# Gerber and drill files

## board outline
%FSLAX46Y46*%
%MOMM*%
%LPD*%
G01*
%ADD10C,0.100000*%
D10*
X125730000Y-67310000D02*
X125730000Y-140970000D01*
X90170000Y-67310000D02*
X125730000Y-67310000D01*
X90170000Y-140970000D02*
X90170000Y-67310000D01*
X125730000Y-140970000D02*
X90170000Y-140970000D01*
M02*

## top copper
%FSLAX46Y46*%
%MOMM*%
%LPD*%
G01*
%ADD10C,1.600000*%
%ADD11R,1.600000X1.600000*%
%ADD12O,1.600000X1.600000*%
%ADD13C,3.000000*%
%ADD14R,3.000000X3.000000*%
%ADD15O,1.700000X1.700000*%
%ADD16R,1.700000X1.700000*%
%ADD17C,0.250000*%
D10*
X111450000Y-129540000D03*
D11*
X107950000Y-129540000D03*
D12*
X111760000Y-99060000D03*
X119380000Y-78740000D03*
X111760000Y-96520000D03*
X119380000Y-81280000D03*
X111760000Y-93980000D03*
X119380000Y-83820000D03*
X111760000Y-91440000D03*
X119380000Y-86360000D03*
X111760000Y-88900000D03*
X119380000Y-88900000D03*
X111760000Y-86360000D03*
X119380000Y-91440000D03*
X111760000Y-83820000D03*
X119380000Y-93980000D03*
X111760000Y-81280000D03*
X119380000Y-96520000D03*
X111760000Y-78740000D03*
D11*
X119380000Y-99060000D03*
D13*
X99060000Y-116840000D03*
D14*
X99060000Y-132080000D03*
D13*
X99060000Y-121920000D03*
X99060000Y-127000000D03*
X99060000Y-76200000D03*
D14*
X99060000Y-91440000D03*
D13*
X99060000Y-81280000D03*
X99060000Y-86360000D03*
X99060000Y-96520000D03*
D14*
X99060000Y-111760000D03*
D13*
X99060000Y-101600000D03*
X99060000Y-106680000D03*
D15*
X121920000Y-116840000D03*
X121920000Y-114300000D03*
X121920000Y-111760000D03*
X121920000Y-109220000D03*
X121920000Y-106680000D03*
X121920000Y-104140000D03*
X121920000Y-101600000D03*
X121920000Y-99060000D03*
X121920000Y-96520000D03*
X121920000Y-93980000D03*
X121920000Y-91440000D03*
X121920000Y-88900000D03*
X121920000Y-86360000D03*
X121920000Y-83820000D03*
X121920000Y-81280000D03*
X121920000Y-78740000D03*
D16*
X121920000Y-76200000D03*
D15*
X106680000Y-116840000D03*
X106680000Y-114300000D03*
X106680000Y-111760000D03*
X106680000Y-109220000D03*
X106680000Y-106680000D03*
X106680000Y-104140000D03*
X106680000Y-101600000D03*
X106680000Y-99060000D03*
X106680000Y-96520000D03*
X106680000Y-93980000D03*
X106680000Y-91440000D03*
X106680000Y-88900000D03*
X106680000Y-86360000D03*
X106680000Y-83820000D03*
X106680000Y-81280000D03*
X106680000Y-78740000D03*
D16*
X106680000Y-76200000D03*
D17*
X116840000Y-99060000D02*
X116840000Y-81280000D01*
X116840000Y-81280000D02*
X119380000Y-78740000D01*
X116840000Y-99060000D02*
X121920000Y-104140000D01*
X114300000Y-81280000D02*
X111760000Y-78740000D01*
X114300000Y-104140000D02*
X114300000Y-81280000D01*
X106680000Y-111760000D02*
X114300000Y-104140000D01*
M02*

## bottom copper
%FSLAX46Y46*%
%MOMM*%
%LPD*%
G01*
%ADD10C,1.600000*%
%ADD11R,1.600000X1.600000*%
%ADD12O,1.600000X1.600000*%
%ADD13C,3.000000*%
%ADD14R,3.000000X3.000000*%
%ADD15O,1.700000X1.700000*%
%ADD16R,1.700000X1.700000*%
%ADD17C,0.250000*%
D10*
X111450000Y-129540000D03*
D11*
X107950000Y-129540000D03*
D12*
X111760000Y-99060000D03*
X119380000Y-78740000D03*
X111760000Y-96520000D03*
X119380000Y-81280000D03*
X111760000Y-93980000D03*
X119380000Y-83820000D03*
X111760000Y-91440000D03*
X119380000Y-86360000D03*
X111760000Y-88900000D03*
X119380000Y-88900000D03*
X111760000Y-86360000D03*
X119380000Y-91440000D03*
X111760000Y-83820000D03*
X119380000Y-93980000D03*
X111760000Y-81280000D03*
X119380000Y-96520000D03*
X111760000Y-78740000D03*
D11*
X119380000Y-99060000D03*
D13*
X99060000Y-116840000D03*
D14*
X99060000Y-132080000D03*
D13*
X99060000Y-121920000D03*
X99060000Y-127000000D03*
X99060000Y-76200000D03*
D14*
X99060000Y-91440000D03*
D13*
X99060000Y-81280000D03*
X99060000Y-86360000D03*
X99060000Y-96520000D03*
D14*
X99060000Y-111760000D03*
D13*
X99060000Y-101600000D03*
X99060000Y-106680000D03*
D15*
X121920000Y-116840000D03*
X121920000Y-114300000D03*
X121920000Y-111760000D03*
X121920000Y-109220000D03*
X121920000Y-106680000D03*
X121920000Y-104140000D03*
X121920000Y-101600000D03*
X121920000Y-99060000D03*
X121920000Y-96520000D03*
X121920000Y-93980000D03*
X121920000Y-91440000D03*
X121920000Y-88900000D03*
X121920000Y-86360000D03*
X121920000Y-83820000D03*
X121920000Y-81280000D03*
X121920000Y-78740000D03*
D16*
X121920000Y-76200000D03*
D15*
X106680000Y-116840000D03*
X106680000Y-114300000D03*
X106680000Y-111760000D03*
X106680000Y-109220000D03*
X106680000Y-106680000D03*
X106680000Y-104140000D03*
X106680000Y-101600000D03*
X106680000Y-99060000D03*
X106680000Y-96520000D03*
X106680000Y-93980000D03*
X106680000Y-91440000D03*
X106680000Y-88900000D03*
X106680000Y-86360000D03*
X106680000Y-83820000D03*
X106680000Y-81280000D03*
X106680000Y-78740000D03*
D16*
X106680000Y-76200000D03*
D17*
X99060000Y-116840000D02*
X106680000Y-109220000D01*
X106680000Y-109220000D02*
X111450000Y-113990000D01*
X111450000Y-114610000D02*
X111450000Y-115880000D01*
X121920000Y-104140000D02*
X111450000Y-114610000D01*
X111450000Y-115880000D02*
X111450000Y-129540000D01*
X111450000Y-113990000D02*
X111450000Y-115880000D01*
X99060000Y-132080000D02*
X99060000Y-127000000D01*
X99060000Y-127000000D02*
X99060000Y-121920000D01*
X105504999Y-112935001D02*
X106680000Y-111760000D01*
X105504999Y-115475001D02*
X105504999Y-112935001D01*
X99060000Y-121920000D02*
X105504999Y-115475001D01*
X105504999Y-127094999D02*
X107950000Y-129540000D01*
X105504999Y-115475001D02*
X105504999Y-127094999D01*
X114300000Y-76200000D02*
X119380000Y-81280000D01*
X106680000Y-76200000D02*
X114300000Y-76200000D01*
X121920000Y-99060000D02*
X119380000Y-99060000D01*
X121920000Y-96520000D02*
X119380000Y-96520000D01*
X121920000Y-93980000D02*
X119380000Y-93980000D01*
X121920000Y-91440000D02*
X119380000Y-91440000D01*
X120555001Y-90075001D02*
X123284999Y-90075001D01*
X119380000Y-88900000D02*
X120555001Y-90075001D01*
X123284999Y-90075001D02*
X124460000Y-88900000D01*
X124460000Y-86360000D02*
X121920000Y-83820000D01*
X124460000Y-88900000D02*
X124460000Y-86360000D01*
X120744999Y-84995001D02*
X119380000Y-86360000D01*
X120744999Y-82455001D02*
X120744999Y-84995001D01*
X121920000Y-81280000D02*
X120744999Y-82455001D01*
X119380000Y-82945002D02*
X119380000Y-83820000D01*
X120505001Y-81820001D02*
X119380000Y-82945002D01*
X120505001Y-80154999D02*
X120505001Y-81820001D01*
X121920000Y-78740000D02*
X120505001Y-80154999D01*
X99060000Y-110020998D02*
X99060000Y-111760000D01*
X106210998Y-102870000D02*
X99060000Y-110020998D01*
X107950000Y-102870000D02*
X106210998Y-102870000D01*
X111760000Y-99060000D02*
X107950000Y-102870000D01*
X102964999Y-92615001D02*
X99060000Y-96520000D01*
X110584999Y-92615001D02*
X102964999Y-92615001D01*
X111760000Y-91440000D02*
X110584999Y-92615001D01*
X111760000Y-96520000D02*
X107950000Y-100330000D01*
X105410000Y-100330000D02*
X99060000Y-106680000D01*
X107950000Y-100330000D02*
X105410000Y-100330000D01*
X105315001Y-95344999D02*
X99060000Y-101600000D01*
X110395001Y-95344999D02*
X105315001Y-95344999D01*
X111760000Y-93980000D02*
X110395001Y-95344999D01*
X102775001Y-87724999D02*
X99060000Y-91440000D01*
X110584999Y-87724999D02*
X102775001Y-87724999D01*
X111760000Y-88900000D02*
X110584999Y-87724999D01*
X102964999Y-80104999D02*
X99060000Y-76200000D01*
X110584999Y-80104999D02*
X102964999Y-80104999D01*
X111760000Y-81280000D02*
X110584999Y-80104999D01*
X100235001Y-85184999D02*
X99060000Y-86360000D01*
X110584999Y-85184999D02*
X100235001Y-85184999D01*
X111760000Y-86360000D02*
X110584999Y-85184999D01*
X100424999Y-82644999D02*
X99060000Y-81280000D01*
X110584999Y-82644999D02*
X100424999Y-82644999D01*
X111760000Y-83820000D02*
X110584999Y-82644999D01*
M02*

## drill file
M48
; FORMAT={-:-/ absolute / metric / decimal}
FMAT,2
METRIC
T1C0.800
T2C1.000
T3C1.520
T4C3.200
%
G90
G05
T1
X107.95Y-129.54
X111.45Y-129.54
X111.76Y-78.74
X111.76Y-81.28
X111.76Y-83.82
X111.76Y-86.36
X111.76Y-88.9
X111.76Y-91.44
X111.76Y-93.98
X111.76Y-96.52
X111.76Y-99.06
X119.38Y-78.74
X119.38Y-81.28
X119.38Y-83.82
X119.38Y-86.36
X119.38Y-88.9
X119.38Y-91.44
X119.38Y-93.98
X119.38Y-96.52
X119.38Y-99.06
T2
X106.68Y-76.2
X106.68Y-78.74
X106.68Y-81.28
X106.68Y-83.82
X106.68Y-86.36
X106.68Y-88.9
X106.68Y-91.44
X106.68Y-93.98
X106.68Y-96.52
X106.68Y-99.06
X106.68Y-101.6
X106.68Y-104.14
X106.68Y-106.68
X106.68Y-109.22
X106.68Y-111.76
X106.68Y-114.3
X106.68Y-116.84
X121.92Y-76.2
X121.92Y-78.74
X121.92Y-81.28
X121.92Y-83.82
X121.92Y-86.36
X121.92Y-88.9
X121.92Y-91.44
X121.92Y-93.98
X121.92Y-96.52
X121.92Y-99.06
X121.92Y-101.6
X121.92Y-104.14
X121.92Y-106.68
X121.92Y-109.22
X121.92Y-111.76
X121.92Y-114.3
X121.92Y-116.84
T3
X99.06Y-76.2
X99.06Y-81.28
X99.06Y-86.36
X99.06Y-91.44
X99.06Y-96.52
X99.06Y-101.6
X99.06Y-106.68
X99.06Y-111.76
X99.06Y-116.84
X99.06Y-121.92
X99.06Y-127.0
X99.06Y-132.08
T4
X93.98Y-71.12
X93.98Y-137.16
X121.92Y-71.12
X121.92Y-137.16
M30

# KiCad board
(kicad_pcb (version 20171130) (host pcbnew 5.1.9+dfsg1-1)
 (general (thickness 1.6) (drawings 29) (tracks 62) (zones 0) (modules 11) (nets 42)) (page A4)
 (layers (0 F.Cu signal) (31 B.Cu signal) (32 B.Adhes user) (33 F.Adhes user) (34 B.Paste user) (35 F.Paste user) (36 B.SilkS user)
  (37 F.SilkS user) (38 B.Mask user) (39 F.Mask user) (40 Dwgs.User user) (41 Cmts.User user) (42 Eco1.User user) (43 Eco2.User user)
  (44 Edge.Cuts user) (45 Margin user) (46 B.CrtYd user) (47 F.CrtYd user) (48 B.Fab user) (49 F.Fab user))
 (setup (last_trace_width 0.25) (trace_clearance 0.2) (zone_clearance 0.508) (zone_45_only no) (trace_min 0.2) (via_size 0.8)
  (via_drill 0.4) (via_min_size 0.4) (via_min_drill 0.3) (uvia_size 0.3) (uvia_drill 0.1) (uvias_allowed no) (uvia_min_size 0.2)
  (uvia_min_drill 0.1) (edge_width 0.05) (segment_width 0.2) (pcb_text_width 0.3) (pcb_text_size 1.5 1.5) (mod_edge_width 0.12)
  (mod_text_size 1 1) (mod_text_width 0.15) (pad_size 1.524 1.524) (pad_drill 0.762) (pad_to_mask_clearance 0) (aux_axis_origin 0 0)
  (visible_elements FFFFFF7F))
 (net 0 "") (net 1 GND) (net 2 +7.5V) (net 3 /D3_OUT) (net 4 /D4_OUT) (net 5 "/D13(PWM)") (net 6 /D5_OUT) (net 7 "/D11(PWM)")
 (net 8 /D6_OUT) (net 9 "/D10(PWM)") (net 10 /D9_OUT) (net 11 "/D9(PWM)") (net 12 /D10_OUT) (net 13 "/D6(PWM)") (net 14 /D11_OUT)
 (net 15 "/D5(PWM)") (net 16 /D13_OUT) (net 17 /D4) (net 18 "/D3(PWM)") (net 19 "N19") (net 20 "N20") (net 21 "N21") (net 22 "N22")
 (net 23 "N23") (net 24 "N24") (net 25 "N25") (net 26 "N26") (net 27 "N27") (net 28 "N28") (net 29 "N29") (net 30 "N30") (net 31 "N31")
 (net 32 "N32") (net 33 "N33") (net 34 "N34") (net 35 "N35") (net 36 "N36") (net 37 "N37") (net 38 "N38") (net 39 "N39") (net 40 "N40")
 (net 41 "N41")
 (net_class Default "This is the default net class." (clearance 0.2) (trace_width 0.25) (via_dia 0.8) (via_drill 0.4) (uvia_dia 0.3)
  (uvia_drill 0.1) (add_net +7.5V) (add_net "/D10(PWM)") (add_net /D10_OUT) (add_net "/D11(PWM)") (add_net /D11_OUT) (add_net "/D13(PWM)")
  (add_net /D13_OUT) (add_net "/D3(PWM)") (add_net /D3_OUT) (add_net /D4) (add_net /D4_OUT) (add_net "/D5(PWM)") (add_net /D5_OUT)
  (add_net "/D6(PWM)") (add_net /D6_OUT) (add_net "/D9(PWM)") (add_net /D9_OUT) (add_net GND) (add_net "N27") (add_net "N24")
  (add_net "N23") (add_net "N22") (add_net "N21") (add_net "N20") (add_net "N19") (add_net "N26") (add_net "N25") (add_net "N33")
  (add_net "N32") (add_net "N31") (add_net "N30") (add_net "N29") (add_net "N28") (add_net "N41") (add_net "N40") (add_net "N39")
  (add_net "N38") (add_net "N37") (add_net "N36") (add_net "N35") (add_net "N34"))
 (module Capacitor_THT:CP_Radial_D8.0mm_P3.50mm (layer F.Cu) (at 107.95 129.54)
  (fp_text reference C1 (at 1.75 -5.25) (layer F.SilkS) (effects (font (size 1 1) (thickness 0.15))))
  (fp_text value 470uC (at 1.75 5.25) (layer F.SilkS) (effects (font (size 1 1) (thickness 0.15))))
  (pad 2 thru_hole circle (at 3.5 0) (size 1.6 1.6) (drill 0.8) (layers *.Cu *.Mask) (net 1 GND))
  (pad 1 thru_hole rect (at 0 0) (size 1.6 1.6) (drill 0.8) (layers *.Cu *.Mask) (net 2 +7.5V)))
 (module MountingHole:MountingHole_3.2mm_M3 (layer F.Cu) (at 121.92 137.16)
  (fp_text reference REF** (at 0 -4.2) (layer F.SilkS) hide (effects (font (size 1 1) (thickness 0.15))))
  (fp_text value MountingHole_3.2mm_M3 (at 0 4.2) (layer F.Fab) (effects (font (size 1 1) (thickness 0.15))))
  (pad 1 np_thru_hole circle (at 0 0) (size 3.2 3.2) (drill 3.2) (layers *.Cu *.Mask)))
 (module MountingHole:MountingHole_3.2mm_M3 (layer F.Cu) (at 93.98 137.16)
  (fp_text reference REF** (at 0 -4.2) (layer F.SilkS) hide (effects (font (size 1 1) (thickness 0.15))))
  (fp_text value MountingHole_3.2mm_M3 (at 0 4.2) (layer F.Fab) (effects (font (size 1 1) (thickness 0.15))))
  (pad 1 np_thru_hole circle (at 0 0) (size 3.2 3.2) (drill 3.2) (layers *.Cu *.Mask)))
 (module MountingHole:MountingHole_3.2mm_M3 (layer F.Cu) (at 121.92 71.12)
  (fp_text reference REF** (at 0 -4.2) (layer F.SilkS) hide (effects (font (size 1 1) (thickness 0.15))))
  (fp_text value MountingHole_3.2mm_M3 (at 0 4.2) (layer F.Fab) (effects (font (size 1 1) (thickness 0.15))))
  (pad 1 np_thru_hole circle (at 0 0) (size 3.2 3.2) (drill 3.2) (layers *.Cu *.Mask)))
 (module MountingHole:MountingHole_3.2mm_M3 (layer F.Cu) (at 93.98 71.12)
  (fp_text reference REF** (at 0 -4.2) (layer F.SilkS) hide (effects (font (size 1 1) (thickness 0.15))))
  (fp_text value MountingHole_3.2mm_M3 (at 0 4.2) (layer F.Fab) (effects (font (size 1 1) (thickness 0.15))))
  (pad 1 np_thru_hole circle (at 0 0) (size 3.2 3.2) (drill 3.2) (layers *.Cu *.Mask)))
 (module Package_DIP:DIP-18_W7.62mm (layer F.Cu) (at 119.38 99.06 180)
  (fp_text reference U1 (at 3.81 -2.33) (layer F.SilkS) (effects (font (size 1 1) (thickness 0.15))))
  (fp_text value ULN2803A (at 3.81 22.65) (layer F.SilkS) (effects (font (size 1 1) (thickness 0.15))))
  (pad 18 thru_hole oval (at 7.62 0 180) (size 1.6 1.6) (drill 0.8) (layers *.Cu *.Mask) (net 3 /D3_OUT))
  (pad 9 thru_hole oval (at 0 20.32 180) (size 1.6 1.6) (drill 0.8) (layers *.Cu *.Mask) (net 1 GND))
  (pad 17 thru_hole oval (at 7.62 2.54 180) (size 1.6 1.6) (drill 0.8) (layers *.Cu *.Mask) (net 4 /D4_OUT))
  (pad 8 thru_hole oval (at 0 17.78 180) (size 1.6 1.6) (drill 0.8) (layers *.Cu *.Mask) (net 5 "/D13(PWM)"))
  (pad 16 thru_hole oval (at 7.62 5.08 180) (size 1.6 1.6) (drill 0.8) (layers *.Cu *.Mask) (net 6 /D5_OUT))
  (pad 7 thru_hole oval (at 0 15.24 180) (size 1.6 1.6) (drill 0.8) (layers *.Cu *.Mask) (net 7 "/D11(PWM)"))
  (pad 15 thru_hole oval (at 7.62 7.62 180) (size 1.6 1.6) (drill 0.8) (layers *.Cu *.Mask) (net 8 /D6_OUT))
  (pad 6 thru_hole oval (at 0 12.7 180) (size 1.6 1.6) (drill 0.8) (layers *.Cu *.Mask) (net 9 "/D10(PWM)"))
  (pad 14 thru_hole oval (at 7.62 10.16 180) (size 1.6 1.6) (drill 0.8) (layers *.Cu *.Mask) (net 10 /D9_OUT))
  (pad 5 thru_hole oval (at 0 10.16 180) (size 1.6 1.6) (drill 0.8) (layers *.Cu *.Mask) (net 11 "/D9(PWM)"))
  (pad 13 thru_hole oval (at 7.62 12.7 180) (size 1.6 1.6) (drill 0.8) (layers *.Cu *.Mask) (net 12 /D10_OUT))
  (pad 4 thru_hole oval (at 0 7.62 180) (size 1.6 1.6) (drill 0.8) (layers *.Cu *.Mask) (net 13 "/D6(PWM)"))
  (pad 12 thru_hole oval (at 7.62 15.24 180) (size 1.6 1.6) (drill 0.8) (layers *.Cu *.Mask) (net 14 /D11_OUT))
  (pad 3 thru_hole oval (at 0 5.08 180) (size 1.6 1.6) (drill 0.8) (layers *.Cu *.Mask) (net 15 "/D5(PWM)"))
  (pad 11 thru_hole oval (at 7.62 17.78 180) (size 1.6 1.6) (drill 0.8) (layers *.Cu *.Mask) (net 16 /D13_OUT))
  (pad 2 thru_hole oval (at 0 2.54 180) (size 1.6 1.6) (drill 0.8) (layers *.Cu *.Mask) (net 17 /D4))
  (pad 10 thru_hole oval (at 7.62 20.32 180) (size 1.6 1.6) (drill 0.8) (layers *.Cu *.Mask) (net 2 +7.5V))
  (pad 1 thru_hole rect (at 0 0 180) (size 1.6 1.6) (drill 0.8) (layers *.Cu *.Mask) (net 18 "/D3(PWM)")))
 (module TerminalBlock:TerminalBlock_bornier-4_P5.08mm (layer F.Cu) (at 99.06 132.08 90)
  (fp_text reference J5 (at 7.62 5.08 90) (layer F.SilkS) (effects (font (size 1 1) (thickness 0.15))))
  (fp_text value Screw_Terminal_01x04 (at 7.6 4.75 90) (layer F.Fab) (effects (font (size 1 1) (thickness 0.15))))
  (pad 4 thru_hole circle (at 15.24 0 90) (size 3 3) (drill 1.52) (layers *.Cu *.Mask) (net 1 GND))
  (pad 1 thru_hole rect (at 0 0 90) (size 3 3) (drill 1.52) (layers *.Cu *.Mask) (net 2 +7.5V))
  (pad 3 thru_hole circle (at 10.16 0 90) (size 3 3) (drill 1.52) (layers *.Cu *.Mask) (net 2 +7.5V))
  (pad 2 thru_hole circle (at 5.08 0 90) (size 3 3) (drill 1.52) (layers *.Cu *.Mask) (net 2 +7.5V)))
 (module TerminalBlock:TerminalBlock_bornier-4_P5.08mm (layer F.Cu) (at 99.06 91.44 90)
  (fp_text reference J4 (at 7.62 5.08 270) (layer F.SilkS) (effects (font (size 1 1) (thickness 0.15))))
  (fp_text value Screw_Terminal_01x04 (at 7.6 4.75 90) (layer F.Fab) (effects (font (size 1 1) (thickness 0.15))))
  (pad 4 thru_hole circle (at 15.24 0 90) (size 3 3) (drill 1.52) (layers *.Cu *.Mask) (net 16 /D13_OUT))
  (pad 1 thru_hole rect (at 0 0 90) (size 3 3) (drill 1.52) (layers *.Cu *.Mask) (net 10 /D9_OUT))
  (pad 3 thru_hole circle (at 10.16 0 90) (size 3 3) (drill 1.52) (layers *.Cu *.Mask) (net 14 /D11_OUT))
  (pad 2 thru_hole circle (at 5.08 0 90) (size 3 3) (drill 1.52) (layers *.Cu *.Mask) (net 12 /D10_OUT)))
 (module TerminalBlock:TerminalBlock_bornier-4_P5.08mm (layer F.Cu) (at 99.06 111.76 90)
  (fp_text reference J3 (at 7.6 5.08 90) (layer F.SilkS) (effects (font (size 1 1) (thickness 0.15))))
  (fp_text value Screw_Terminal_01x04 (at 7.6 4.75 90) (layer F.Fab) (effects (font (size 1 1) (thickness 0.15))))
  (pad 4 thru_hole circle (at 15.24 0 90) (size 3 3) (drill 1.52) (layers *.Cu *.Mask) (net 8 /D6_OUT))
  (pad 1 thru_hole rect (at 0 0 90) (size 3 3) (drill 1.52) (layers *.Cu *.Mask) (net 3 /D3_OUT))
  (pad 3 thru_hole circle (at 10.16 0 90) (size 3 3) (drill 1.52) (layers *.Cu *.Mask) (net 6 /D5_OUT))
  (pad 2 thru_hole circle (at 5.08 0 90) (size 3 3) (drill 1.52) (layers *.Cu *.Mask) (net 4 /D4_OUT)))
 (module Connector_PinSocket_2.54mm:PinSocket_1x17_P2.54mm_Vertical (layer F.Cu) (at 121.92 76.2)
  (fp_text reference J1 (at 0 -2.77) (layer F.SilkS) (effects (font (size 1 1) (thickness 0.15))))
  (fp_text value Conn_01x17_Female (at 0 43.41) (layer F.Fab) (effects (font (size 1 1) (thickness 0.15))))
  (pad 17 thru_hole oval (at 0 40.64) (size 1.7 1.7) (drill 1) (layers *.Cu *.Mask) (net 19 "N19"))
  (pad 16 thru_hole oval (at 0 38.1) (size 1.7 1.7) (drill 1) (layers *.Cu *.Mask) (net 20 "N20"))
  (pad 15 thru_hole oval (at 0 35.56) (size 1.7 1.7) (drill 1) (layers *.Cu *.Mask) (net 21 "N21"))
  (pad 14 thru_hole oval (at 0 33.02) (size 1.7 1.7) (drill 1) (layers *.Cu *.Mask) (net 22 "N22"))
  (pad 13 thru_hole oval (at 0 30.48) (size 1.7 1.7) (drill 1) (layers *.Cu *.Mask) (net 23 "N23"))
  (pad 12 thru_hole oval (at 0 27.94) (size 1.7 1.7) (drill 1) (layers *.Cu *.Mask) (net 1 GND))
  (pad 11 thru_hole oval (at 0 25.4) (size 1.7 1.7) (drill 1) (layers *.Cu *.Mask) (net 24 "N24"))
  (pad 10 thru_hole oval (at 0 22.86) (size 1.7 1.7) (drill 1) (layers *.Cu *.Mask) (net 18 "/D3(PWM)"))
  (pad 9 thru_hole oval (at 0 20.32) (size 1.7 1.7) (drill 1) (layers *.Cu *.Mask) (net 17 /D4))
  (pad 8 thru_hole oval (at 0 17.78) (size 1.7 1.7) (drill 1) (layers *.Cu *.Mask) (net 15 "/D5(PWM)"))
  (pad 7 thru_hole oval (at 0 15.24) (size 1.7 1.7) (drill 1) (layers *.Cu *.Mask) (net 13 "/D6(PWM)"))
  (pad 6 thru_hole oval (at 0 12.7) (size 1.7 1.7) (drill 1) (layers *.Cu *.Mask) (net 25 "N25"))
  (pad 5 thru_hole oval (at 0 10.16) (size 1.7 1.7) (drill 1) (layers *.Cu *.Mask) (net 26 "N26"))
  (pad 4 thru_hole oval (at 0 7.62) (size 1.7 1.7) (drill 1) (layers *.Cu *.Mask) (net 11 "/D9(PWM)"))
  (pad 3 thru_hole oval (at 0 5.08) (size 1.7 1.7) (drill 1) (layers *.Cu *.Mask) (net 9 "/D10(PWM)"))
  (pad 2 thru_hole oval (at 0 2.54) (size 1.7 1.7) (drill 1) (layers *.Cu *.Mask) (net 7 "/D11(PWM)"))
  (pad 1 thru_hole rect (at 0 0) (size 1.7 1.7) (drill 1) (layers *.Cu *.Mask) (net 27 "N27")))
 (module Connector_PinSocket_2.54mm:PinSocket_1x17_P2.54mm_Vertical (layer F.Cu) (at 106.68 76.2)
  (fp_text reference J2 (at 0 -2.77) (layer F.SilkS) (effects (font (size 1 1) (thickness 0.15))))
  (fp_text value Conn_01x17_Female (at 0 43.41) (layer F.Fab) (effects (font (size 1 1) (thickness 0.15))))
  (pad 17 thru_hole oval (at 0 40.64) (size 1.7 1.7) (drill 1) (layers *.Cu *.Mask) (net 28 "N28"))
  (pad 16 thru_hole oval (at 0 38.1) (size 1.7 1.7) (drill 1) (layers *.Cu *.Mask) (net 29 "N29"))
  (pad 15 thru_hole oval (at 0 35.56) (size 1.7 1.7) (drill 1) (layers *.Cu *.Mask) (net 2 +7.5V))
  (pad 14 thru_hole oval (at 0 33.02) (size 1.7 1.7) (drill 1) (layers *.Cu *.Mask) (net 1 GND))
  (pad 13 thru_hole oval (at 0 30.48) (size 1.7 1.7) (drill 1) (layers *.Cu *.Mask) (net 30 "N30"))
  (pad 12 thru_hole oval (at 0 27.94) (size 1.7 1.7) (drill 1) (layers *.Cu *.Mask) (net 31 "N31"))
  (pad 11 thru_hole oval (at 0 25.4) (size 1.7 1.7) (drill 1) (layers *.Cu *.Mask) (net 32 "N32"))
  (pad 10 thru_hole oval (at 0 22.86) (size 1.7 1.7) (drill 1) (layers *.Cu *.Mask) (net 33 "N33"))
  (pad 9 thru_hole oval (at 0 20.32) (size 1.7 1.7) (drill 1) (layers *.Cu *.Mask) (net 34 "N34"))
  (pad 8 thru_hole oval (at 0 17.78) (size 1.7 1.7) (drill 1) (layers *.Cu *.Mask) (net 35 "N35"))
  (pad 7 thru_hole oval (at 0 15.24) (size 1.7 1.7) (drill 1) (layers *.Cu *.Mask) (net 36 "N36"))
  (pad 6 thru_hole oval (at 0 12.7) (size 1.7 1.7) (drill 1) (layers *.Cu *.Mask) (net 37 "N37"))
  (pad 5 thru_hole oval (at 0 10.16) (size 1.7 1.7) (drill 1) (layers *.Cu *.Mask) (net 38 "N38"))
  (pad 4 thru_hole oval (at 0 7.62) (size 1.7 1.7) (drill 1) (layers *.Cu *.Mask) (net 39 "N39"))
  (pad 3 thru_hole oval (at 0 5.08) (size 1.7 1.7) (drill 1) (layers *.Cu *.Mask) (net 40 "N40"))
  (pad 2 thru_hole oval (at 0 2.54) (size 1.7 1.7) (drill 1) (layers *.Cu *.Mask) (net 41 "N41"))
  (pad 1 thru_hole rect (at 0 0) (size 1.7 1.7) (drill 1) (layers *.Cu *.Mask) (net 5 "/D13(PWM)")))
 (gr_line (start 125.73 67.31) (end 125.73 140.97) (layer Edge.Cuts) (width 0.1))
 (gr_line (start 90.17 67.31) (end 125.73 67.31) (layer Edge.Cuts) (width 0.1))
 (gr_line (start 90.17 140.97) (end 90.17 67.31) (layer Edge.Cuts) (width 0.1))
 (gr_line (start 125.73 140.97) (end 90.17 140.97) (layer Edge.Cuts) (width 0.1))
 (segment (start 99.06 116.84) (end 106.68 109.22) (width 0.25) (layer B.Cu) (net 1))
 (segment (start 116.84 99.06) (end 116.84 81.28) (width 0.25) (layer F.Cu) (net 1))
 (segment (start 116.84 81.28) (end 119.38 78.74) (width 0.25) (layer F.Cu) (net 1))
 (segment (start 116.84 99.06) (end 121.92 104.14) (width 0.25) (layer F.Cu) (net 1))
 (segment (start 106.68 109.22) (end 111.45 113.99) (width 0.25) (layer B.Cu) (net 1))
 (segment (start 111.45 114.61) (end 111.45 115.88) (width 0.25) (layer B.Cu) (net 1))
 (segment (start 121.92 104.14) (end 111.45 114.61) (width 0.25) (layer B.Cu) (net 1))
 (segment (start 111.45 115.88) (end 111.45 129.54) (width 0.25) (layer B.Cu) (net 1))
 (segment (start 111.45 113.99) (end 111.45 115.88) (width 0.25) (layer B.Cu) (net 1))
 (segment (start 99.06 132.08) (end 99.06 127) (width 0.25) (layer B.Cu) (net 2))
 (segment (start 99.06 127) (end 99.06 121.92) (width 0.25) (layer B.Cu) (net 2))
 (segment (start 105.504999 112.935001) (end 106.68 111.76) (width 0.25) (layer B.Cu) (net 2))
 (segment (start 105.504999 115.475001) (end 105.504999 112.935001) (width 0.25) (layer B.Cu) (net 2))
 (segment (start 114.3 81.28) (end 111.76 78.74) (width 0.25) (layer F.Cu) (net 2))
 (segment (start 114.3 104.14) (end 114.3 81.28) (width 0.25) (layer F.Cu) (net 2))
 (segment (start 106.68 111.76) (end 114.3 104.14) (width 0.25) (layer F.Cu) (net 2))
 (segment (start 99.06 121.92) (end 105.504999 115.475001) (width 0.25) (layer B.Cu) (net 2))
 (segment (start 105.504999 127.094999) (end 107.95 129.54) (width 0.25) (layer B.Cu) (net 2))
 (segment (start 105.504999 115.475001) (end 105.504999 127.094999) (width 0.25) (layer B.Cu) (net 2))
 (segment (start 114.3 76.2) (end 119.38 81.28) (width 0.25) (layer B.Cu) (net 5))
 (segment (start 106.68 76.2) (end 114.3 76.2) (width 0.25) (layer B.Cu) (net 5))
 (segment (start 121.92 99.06) (end 119.38 99.06) (width 0.25) (layer B.Cu) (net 18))
 (segment (start 121.92 96.52) (end 119.38 96.52) (width 0.25) (layer B.Cu) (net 17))
 (segment (start 121.92 93.98) (end 119.38 93.98) (width 0.25) (layer B.Cu) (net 15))
 (segment (start 121.92 91.44) (end 119.38 91.44) (width 0.25) (layer B.Cu) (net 13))
 (segment (start 120.555001 90.075001) (end 123.284999 90.075001) (width 0.25) (layer B.Cu) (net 11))
 (segment (start 119.38 88.9) (end 120.555001 90.075001) (width 0.25) (layer B.Cu) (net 11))
 (segment (start 123.284999 90.075001) (end 124.46 88.9) (width 0.25) (layer B.Cu) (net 11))
 (segment (start 124.46 86.36) (end 121.92 83.82) (width 0.25) (layer B.Cu) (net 11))
 (segment (start 124.46 88.9) (end 124.46 86.36) (width 0.25) (layer B.Cu) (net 11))
 (segment (start 120.744999 84.995001) (end 119.38 86.36) (width 0.25) (layer B.Cu) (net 9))
 (segment (start 120.744999 82.455001) (end 120.744999 84.995001) (width 0.25) (layer B.Cu) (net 9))
 (segment (start 121.92 81.28) (end 120.744999 82.455001) (width 0.25) (layer B.Cu) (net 9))
 (segment (start 119.38 82.945002) (end 119.38 83.82) (width 0.25) (layer B.Cu) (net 7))
 (segment (start 120.505001 81.820001) (end 119.38 82.945002) (width 0.25) (layer B.Cu) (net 7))
 (segment (start 120.505001 80.154999) (end 120.505001 81.820001) (width 0.25) (layer B.Cu) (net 7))
 (segment (start 121.92 78.74) (end 120.505001 80.154999) (width 0.25) (layer B.Cu) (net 7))
 (segment (start 99.06 110.020998) (end 99.06 111.76) (width 0.25) (layer B.Cu) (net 3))
 (segment (start 106.210998 102.87) (end 99.06 110.020998) (width 0.25) (layer B.Cu) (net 3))
 (segment (start 107.95 102.87) (end 106.210998 102.87) (width 0.25) (layer B.Cu) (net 3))
 (segment (start 111.76 99.06) (end 107.95 102.87) (width 0.25) (layer B.Cu) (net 3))
 (segment (start 102.964999 92.615001) (end 99.06 96.52) (width 0.25) (layer B.Cu) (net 8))
 (segment (start 110.584999 92.615001) (end 102.964999 92.615001) (width 0.25) (layer B.Cu) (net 8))
 (segment (start 111.76 91.44) (end 110.584999 92.615001) (width 0.25) (layer B.Cu) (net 8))
 (segment (start 111.76 96.52) (end 107.95 100.33) (width 0.25) (layer B.Cu) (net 4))
 (segment (start 105.41 100.33) (end 99.06 106.68) (width 0.25) (layer B.Cu) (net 4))
 (segment (start 107.95 100.33) (end 105.41 100.33) (width 0.25) (layer B.Cu) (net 4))
 (segment (start 105.315001 95.344999) (end 99.06 101.6) (width 0.25) (layer B.Cu) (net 6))
 (segment (start 110.395001 95.344999) (end 105.315001 95.344999) (width 0.25) (layer B.Cu) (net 6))
 (segment (start 111.76 93.98) (end 110.395001 95.344999) (width 0.25) (layer B.Cu) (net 6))
 (segment (start 102.775001 87.724999) (end 99.06 91.44) (width 0.25) (layer B.Cu) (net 10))
 (segment (start 110.584999 87.724999) (end 102.775001 87.724999) (width 0.25) (layer B.Cu) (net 10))
 (segment (start 111.76 88.9) (end 110.584999 87.724999) (width 0.25) (layer B.Cu) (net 10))
 (segment (start 102.964999 80.104999) (end 99.06 76.2) (width 0.25) (layer B.Cu) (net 16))
 (segment (start 110.584999 80.104999) (end 102.964999 80.104999) (width 0.25) (layer B.Cu) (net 16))
 (segment (start 111.76 81.28) (end 110.584999 80.104999) (width 0.25) (layer B.Cu) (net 16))
 (segment (start 100.235001 85.184999) (end 99.06 86.36) (width 0.25) (layer B.Cu) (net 12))
 (segment (start 110.584999 85.184999) (end 100.235001 85.184999) (width 0.25) (layer B.Cu) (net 12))
 (segment (start 111.76 86.36) (end 110.584999 85.184999) (width 0.25) (layer B.Cu) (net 12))
 (segment (start 100.424999 82.644999) (end 99.06 81.28) (width 0.25) (layer B.Cu) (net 14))
 (segment (start 110.584999 82.644999) (end 100.424999 82.644999) (width 0.25) (layer B.Cu) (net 14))
 (segment (start 111.76 83.82) (end 110.584999 82.644999) (width 0.25) (layer B.Cu) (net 14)))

